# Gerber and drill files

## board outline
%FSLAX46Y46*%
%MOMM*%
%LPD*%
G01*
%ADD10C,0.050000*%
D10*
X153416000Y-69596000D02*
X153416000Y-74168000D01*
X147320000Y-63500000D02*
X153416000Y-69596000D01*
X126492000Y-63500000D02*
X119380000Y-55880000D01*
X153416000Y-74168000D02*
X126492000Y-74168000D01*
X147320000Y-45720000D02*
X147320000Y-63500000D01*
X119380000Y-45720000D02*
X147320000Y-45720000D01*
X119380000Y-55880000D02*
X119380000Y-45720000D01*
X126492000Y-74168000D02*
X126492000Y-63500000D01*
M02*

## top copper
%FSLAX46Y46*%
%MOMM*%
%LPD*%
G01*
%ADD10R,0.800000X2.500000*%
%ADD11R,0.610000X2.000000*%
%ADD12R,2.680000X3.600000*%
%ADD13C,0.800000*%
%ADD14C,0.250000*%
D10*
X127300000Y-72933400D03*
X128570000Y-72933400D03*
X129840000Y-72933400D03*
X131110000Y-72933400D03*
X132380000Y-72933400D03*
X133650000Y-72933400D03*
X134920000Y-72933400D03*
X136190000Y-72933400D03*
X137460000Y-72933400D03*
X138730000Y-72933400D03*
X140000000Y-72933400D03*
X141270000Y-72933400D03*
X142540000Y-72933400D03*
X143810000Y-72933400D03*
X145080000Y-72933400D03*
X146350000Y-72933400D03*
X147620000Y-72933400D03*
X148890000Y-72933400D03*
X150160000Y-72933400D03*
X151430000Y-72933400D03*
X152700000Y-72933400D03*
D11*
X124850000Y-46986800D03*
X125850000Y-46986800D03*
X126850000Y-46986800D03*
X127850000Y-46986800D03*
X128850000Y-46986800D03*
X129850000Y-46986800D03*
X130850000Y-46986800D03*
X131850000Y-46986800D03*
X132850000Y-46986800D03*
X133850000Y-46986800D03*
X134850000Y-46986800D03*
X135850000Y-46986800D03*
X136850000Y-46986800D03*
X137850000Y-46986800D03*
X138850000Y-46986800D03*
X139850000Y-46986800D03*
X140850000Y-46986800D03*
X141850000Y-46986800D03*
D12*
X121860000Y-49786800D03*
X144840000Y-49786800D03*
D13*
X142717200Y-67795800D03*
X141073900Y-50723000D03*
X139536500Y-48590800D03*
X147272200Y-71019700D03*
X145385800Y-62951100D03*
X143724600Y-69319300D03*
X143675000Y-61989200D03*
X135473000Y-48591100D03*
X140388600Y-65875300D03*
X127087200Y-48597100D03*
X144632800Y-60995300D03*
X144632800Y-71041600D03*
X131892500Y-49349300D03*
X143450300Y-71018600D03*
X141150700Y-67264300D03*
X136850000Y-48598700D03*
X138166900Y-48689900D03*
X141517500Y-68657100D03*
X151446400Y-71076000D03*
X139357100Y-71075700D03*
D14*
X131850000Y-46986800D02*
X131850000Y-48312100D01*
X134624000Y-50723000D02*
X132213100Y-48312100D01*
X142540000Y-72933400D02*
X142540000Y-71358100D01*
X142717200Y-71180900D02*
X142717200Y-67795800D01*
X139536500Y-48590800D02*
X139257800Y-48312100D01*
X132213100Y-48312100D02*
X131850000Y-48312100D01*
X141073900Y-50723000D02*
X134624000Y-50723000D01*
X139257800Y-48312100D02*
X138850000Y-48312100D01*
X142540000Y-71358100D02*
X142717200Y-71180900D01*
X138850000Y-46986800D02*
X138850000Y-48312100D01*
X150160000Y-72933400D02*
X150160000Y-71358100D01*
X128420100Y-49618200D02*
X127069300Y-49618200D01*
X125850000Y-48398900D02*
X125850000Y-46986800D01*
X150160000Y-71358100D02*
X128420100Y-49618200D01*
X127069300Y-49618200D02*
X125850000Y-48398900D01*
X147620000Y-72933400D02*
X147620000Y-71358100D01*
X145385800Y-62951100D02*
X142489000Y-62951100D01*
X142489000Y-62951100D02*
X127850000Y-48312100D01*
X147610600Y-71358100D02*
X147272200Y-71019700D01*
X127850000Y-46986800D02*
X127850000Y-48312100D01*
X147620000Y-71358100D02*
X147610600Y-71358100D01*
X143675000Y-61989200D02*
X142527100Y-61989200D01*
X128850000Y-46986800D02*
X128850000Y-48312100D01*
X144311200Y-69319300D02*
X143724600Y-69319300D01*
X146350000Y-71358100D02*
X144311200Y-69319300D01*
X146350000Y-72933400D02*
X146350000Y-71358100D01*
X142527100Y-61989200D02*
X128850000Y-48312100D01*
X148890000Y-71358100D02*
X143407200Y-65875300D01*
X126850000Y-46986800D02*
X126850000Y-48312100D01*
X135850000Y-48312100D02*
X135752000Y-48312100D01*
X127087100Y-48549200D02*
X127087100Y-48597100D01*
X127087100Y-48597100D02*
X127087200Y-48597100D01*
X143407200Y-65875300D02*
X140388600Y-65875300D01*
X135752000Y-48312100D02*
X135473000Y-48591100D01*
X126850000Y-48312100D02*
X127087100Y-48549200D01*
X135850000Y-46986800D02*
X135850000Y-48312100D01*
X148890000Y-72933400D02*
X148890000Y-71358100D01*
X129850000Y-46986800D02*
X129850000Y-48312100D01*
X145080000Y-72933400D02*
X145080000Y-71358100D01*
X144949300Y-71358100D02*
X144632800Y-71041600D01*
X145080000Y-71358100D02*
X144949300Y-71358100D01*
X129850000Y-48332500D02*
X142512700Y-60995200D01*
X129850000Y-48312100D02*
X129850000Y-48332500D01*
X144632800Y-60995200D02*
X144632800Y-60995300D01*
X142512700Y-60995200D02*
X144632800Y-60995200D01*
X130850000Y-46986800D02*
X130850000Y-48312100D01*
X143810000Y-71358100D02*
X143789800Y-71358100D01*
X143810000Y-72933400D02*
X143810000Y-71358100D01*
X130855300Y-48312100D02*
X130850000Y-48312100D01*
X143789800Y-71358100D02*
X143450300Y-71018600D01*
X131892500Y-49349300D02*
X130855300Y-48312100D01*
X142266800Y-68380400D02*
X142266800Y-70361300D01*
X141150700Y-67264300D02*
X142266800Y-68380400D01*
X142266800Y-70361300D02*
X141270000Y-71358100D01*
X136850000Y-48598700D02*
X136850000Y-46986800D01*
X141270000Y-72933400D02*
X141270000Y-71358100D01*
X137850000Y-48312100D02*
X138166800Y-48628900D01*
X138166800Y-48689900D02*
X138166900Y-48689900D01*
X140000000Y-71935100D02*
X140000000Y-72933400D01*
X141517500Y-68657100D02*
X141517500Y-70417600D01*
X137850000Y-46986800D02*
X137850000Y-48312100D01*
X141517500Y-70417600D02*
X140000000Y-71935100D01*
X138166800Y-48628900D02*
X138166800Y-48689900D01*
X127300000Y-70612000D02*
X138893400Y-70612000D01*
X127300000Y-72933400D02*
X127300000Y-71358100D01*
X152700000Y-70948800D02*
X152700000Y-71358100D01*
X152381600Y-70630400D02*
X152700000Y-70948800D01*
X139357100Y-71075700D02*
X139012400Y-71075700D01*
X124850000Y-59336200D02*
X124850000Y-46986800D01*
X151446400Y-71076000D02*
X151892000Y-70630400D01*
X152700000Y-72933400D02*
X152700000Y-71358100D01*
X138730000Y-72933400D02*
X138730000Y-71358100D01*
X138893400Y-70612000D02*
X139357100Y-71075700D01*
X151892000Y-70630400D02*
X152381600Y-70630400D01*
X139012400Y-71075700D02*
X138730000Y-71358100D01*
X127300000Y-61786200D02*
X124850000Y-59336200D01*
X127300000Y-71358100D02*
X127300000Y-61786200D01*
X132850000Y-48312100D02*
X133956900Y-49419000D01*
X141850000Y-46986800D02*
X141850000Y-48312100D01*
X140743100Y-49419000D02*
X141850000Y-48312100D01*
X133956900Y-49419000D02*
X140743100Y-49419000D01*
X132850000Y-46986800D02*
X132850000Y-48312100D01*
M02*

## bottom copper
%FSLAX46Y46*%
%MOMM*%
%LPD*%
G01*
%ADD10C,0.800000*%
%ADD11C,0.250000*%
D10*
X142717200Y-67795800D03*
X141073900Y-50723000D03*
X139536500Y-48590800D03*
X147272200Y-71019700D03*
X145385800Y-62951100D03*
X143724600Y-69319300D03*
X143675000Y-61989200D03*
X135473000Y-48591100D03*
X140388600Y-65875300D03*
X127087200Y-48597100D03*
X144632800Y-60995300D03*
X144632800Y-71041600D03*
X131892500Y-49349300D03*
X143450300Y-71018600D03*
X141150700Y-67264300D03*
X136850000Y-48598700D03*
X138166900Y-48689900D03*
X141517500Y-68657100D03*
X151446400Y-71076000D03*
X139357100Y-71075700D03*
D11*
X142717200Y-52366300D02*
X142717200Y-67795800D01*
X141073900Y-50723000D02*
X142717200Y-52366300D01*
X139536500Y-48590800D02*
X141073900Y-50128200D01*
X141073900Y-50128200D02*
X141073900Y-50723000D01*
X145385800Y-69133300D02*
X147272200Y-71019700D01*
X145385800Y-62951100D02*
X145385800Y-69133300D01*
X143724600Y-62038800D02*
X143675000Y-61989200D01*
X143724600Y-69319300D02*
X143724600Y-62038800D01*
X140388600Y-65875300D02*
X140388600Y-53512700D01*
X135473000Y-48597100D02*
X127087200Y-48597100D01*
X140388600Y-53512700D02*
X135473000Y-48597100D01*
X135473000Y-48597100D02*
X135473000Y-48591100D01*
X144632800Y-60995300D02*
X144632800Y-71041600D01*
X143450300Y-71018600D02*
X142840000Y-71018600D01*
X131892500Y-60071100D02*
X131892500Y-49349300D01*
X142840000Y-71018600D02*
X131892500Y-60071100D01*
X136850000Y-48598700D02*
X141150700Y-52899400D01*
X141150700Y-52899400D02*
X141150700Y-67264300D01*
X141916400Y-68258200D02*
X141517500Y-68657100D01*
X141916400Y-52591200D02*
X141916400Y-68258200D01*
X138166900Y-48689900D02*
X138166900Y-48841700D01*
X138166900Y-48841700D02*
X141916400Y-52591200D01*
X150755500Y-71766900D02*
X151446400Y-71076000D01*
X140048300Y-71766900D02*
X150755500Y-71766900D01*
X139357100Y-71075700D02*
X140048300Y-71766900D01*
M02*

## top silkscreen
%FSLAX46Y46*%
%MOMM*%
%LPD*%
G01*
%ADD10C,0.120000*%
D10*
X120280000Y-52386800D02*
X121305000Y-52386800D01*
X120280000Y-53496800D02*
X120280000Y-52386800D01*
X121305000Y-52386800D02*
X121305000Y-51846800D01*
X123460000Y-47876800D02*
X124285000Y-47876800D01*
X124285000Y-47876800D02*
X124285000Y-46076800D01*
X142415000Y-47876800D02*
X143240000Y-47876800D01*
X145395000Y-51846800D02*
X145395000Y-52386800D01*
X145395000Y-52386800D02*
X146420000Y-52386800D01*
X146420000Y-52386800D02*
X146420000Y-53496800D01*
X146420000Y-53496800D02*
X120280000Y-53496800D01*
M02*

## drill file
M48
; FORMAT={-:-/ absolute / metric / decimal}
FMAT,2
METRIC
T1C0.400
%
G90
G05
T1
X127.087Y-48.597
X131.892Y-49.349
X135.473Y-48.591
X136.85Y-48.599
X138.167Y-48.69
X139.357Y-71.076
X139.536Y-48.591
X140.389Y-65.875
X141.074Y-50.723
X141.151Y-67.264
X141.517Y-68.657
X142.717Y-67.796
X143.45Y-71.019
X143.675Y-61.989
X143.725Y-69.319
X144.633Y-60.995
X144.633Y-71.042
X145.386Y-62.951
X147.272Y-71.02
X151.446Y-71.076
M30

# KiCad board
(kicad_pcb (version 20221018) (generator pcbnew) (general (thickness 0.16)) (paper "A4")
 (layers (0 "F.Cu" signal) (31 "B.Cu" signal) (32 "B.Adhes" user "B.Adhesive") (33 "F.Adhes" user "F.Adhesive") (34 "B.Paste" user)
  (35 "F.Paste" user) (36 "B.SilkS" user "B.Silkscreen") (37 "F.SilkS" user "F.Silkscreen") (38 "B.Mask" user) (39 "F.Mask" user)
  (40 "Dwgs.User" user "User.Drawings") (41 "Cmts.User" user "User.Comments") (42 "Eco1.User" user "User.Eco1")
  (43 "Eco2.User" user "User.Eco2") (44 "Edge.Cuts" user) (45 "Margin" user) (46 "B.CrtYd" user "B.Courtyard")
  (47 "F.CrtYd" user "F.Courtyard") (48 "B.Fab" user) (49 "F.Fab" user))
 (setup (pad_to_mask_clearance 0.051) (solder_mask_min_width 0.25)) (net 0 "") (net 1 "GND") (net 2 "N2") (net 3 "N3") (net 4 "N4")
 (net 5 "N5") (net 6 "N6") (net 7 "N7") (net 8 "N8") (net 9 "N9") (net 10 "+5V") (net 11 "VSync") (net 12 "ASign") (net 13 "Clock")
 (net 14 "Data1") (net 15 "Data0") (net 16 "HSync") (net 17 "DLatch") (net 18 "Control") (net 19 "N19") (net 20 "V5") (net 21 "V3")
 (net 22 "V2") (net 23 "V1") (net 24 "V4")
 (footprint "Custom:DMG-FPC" (layer "F.Cu") (at 140 72.9334)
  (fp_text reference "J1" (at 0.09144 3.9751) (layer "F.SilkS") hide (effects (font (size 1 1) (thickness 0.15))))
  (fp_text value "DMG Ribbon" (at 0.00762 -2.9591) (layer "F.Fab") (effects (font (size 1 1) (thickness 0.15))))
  (pad "1" smd rect (at -12.7 0) (size 0.8 2.5) (layers "F.Cu" "F.Paste" "F.Mask") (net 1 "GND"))
  (pad "2" smd rect (at -11.43 0) (size 0.8 2.5) (layers "F.Cu" "F.Paste" "F.Mask") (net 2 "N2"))
  (pad "3" smd rect (at -10.16 0) (size 0.8 2.5) (layers "F.Cu" "F.Paste" "F.Mask") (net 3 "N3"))
  (pad "4" smd rect (at -8.89 0) (size 0.8 2.5) (layers "F.Cu" "F.Paste" "F.Mask") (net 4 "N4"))
  (pad "5" smd rect (at -7.62 0) (size 0.8 2.5) (layers "F.Cu" "F.Paste" "F.Mask") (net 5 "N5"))
  (pad "6" smd rect (at -6.35 0) (size 0.8 2.5) (layers "F.Cu" "F.Paste" "F.Mask") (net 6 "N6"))
  (pad "7" smd rect (at -5.08 0) (size 0.8 2.5) (layers "F.Cu" "F.Paste" "F.Mask") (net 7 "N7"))
  (pad "8" smd rect (at -3.81 0) (size 0.8 2.5) (layers "F.Cu" "F.Paste" "F.Mask") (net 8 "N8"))
  (pad "9" smd rect (at -2.54 0) (size 0.8 2.5) (layers "F.Cu" "F.Paste" "F.Mask") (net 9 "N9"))
  (pad "10" smd rect (at -1.27 0) (size 0.8 2.5) (layers "F.Cu" "F.Paste" "F.Mask") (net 1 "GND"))
  (pad "11" smd rect (at 0 0) (size 0.8 2.5) (layers "F.Cu" "F.Paste" "F.Mask") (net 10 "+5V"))
  (pad "12" smd rect (at 1.27 0) (size 0.8 2.5) (layers "F.Cu" "F.Paste" "F.Mask") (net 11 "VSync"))
  (pad "13" smd rect (at 2.54 0) (size 0.8 2.5) (layers "F.Cu" "F.Paste" "F.Mask") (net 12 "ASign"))
  (pad "14" smd rect (at 3.81 0) (size 0.8 2.5) (layers "F.Cu" "F.Paste" "F.Mask") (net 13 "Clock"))
  (pad "15" smd rect (at 5.08 0) (size 0.8 2.5) (layers "F.Cu" "F.Paste" "F.Mask") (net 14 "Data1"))
  (pad "16" smd rect (at 6.35 0) (size 0.8 2.5) (layers "F.Cu" "F.Paste" "F.Mask") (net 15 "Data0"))
  (pad "17" smd rect (at 7.62 0) (size 0.8 2.5) (layers "F.Cu" "F.Paste" "F.Mask") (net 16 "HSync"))
  (pad "18" smd rect (at 8.89 0) (size 0.8 2.5) (layers "F.Cu" "F.Paste" "F.Mask") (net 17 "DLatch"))
  (pad "19" smd rect (at 10.16 0) (size 0.8 2.5) (layers "F.Cu" "F.Paste" "F.Mask") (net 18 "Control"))
  (pad "20" smd rect (at 11.43 0) (size 0.8 2.5) (layers "F.Cu" "F.Paste" "F.Mask") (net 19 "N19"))
  (pad "21" smd rect (at 12.7 0) (size 0.8 2.5) (layers "F.Cu" "F.Paste" "F.Mask") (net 1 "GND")))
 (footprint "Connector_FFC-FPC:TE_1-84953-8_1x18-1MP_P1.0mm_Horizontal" (layer "F.Cu") (at 133.35 48.7868)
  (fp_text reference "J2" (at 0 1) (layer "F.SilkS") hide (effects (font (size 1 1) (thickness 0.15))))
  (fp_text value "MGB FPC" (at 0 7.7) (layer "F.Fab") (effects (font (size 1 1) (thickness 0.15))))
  (fp_line (start -13.07 3.6) (end -12.045 3.6) (stroke (width 0.12) (type solid)) (layer "F.SilkS"))
  (fp_line (start -13.07 4.71) (end -13.07 3.6) (stroke (width 0.12) (type solid)) (layer "F.SilkS"))
  (fp_line (start -12.045 3.6) (end -12.045 3.06) (stroke (width 0.12) (type solid)) (layer "F.SilkS"))
  (fp_line (start -9.89 -0.91) (end -9.065 -0.91) (stroke (width 0.12) (type solid)) (layer "F.SilkS"))
  (fp_line (start -9.065 -0.91) (end -9.065 -2.71) (stroke (width 0.12) (type solid)) (layer "F.SilkS"))
  (fp_line (start 9.065 -0.91) (end 9.89 -0.91) (stroke (width 0.12) (type solid)) (layer "F.SilkS"))
  (fp_line (start 12.045 3.06) (end 12.045 3.6) (stroke (width 0.12) (type solid)) (layer "F.SilkS"))
  (fp_line (start 12.045 3.6) (end 13.07 3.6) (stroke (width 0.12) (type solid)) (layer "F.SilkS"))
  (fp_line (start 13.07 3.6) (end 13.07 4.71) (stroke (width 0.12) (type solid)) (layer "F.SilkS"))
  (fp_line (start 13.07 4.71) (end -13.07 4.71) (stroke (width 0.12) (type solid)) (layer "F.SilkS"))
  (pad "1" smd rect (at -8.5 -1.8) (size 0.61 2) (layers "F.Cu" "F.Paste" "F.Mask") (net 1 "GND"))
  (pad "2" smd rect (at -7.5 -1.8) (size 0.61 2) (layers "F.Cu" "F.Paste" "F.Mask") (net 18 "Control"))
  (pad "3" smd rect (at -6.5 -1.8) (size 0.61 2) (layers "F.Cu" "F.Paste" "F.Mask") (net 17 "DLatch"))
  (pad "4" smd rect (at -5.5 -1.8) (size 0.61 2) (layers "F.Cu" "F.Paste" "F.Mask") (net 16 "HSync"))
  (pad "5" smd rect (at -4.5 -1.8) (size 0.61 2) (layers "F.Cu" "F.Paste" "F.Mask") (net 15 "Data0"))
  (pad "6" smd rect (at -3.5 -1.8) (size 0.61 2) (layers "F.Cu" "F.Paste" "F.Mask") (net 14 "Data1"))
  (pad "7" smd rect (at -2.5 -1.8) (size 0.61 2) (layers "F.Cu" "F.Paste" "F.Mask") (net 13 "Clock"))
  (pad "8" smd rect (at -1.5 -1.8) (size 0.61 2) (layers "F.Cu" "F.Paste" "F.Mask") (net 12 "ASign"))
  (pad "9" smd rect (at -0.5 -1.8) (size 0.61 2) (layers "F.Cu" "F.Paste" "F.Mask") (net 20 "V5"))
  (pad "10" smd rect (at 0.5 -1.8) (size 0.61 2) (layers "F.Cu" "F.Paste" "F.Mask") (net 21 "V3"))
  (pad "11" smd rect (at 1.5 -1.8) (size 0.61 2) (layers "F.Cu" "F.Paste" "F.Mask") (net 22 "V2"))
  (pad "12" smd rect (at 2.5 -1.8) (size 0.61 2) (layers "F.Cu" "F.Paste" "F.Mask") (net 17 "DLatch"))
  (pad "13" smd rect (at 3.5 -1.8) (size 0.61 2) (layers "F.Cu" "F.Paste" "F.Mask") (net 11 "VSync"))
  (pad "14" smd rect (at 4.5 -1.8) (size 0.61 2) (layers "F.Cu" "F.Paste" "F.Mask") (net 10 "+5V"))
  (pad "15" smd rect (at 5.5 -1.8) (size 0.61 2) (layers "F.Cu" "F.Paste" "F.Mask") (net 12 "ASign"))
  (pad "16" smd rect (at 6.5 -1.8) (size 0.61 2) (layers "F.Cu" "F.Paste" "F.Mask") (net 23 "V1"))
  (pad "17" smd rect (at 7.5 -1.8) (size 0.61 2) (layers "F.Cu" "F.Paste" "F.Mask") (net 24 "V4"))
  (pad "18" smd rect (at 8.5 -1.8) (size 0.61 2) (layers "F.Cu" "F.Paste" "F.Mask") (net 20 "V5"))
  (pad "MP" smd rect (at -11.49 1) (size 2.68 3.6) (layers "F.Cu" "F.Paste" "F.Mask"))
  (pad "MP" smd rect (at 11.49 1) (size 2.68 3.6) (layers "F.Cu" "F.Paste" "F.Mask")))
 (gr_line (start 153.416 69.596) (end 153.416 74.168) (stroke (width 0.05) (type solid)) (layer "Edge.Cuts"))
 (gr_line (start 147.32 63.5) (end 153.416 69.596) (stroke (width 0.05) (type solid)) (layer "Edge.Cuts"))
 (gr_line (start 126.492 63.5) (end 119.38 55.88) (stroke (width 0.05) (type solid)) (layer "Edge.Cuts"))
 (gr_line (start 153.416 74.168) (end 126.492 74.168) (stroke (width 0.05) (type solid)) (layer "Edge.Cuts"))
 (gr_line (start 147.32 45.72) (end 147.32 63.5) (stroke (width 0.05) (type solid)) (layer "Edge.Cuts"))
 (gr_line (start 119.38 45.72) (end 147.32 45.72) (stroke (width 0.05) (type solid)) (layer "Edge.Cuts"))
 (gr_line (start 119.38 55.88) (end 119.38 45.72) (stroke (width 0.05) (type solid)) (layer "Edge.Cuts"))
 (gr_line (start 126.492 74.168) (end 126.492 63.5) (stroke (width 0.05) (type solid)) (layer "Edge.Cuts"))
 (segment (start 131.85 46.9868) (end 131.85 48.3121) (width 0.25) (layer "F.Cu") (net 12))
 (segment (start 134.624 50.723) (end 132.2131 48.3121) (width 0.25) (layer "F.Cu") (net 12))
 (segment (start 142.54 72.9334) (end 142.54 71.3581) (width 0.25) (layer "F.Cu") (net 12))
 (segment (start 142.7172 71.1809) (end 142.7172 67.7958) (width 0.25) (layer "F.Cu") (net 12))
 (segment (start 139.5365 48.5908) (end 139.2578 48.3121) (width 0.25) (layer "F.Cu") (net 12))
 (segment (start 132.2131 48.3121) (end 131.85 48.3121) (width 0.25) (layer "F.Cu") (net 12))
 (segment (start 141.0739 50.723) (end 134.624 50.723) (width 0.25) (layer "F.Cu") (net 12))
 (segment (start 139.2578 48.3121) (end 138.85 48.3121) (width 0.25) (layer "F.Cu") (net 12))
 (segment (start 142.54 71.3581) (end 142.7172 71.1809) (width 0.25) (layer "F.Cu") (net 12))
 (segment (start 138.85 46.9868) (end 138.85 48.3121) (width 0.25) (layer "F.Cu") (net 12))
 (via (at 142.7172 67.7958) (size 0.8) (drill 0.4) (layers "F.Cu" "B.Cu") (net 12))
 (via (at 141.0739 50.723) (size 0.8) (drill 0.4) (layers "F.Cu" "B.Cu") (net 12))
 (via (at 139.5365 48.5908) (size 0.8) (drill 0.4) (layers "F.Cu" "B.Cu") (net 12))
 (segment (start 142.7172 52.3663) (end 142.7172 67.7958) (width 0.25) (layer "B.Cu") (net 12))
 (segment (start 141.0739 50.723) (end 142.7172 52.3663) (width 0.25) (layer "B.Cu") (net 12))
 (segment (start 139.5365 48.5908) (end 141.0739 50.1282) (width 0.25) (layer "B.Cu") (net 12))
 (segment (start 141.0739 50.1282) (end 141.0739 50.723) (width 0.25) (layer "B.Cu") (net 12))
 (segment (start 150.16 72.9334) (end 150.16 71.3581) (width 0.25) (layer "F.Cu") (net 18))
 (segment (start 128.4201 49.6182) (end 127.0693 49.6182) (width 0.25) (layer "F.Cu") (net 18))
 (segment (start 125.85 48.3989) (end 125.85 46.9868) (width 0.25) (layer "F.Cu") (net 18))
 (segment (start 150.16 71.3581) (end 128.4201 49.6182) (width 0.25) (layer "F.Cu") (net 18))
 (segment (start 127.0693 49.6182) (end 125.85 48.3989) (width 0.25) (layer "F.Cu") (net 18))
 (segment (start 147.62 72.9334) (end 147.62 71.3581) (width 0.25) (layer "F.Cu") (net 16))
 (segment (start 145.3858 62.9511) (end 142.489 62.9511) (width 0.25) (layer "F.Cu") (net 16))
 (segment (start 142.489 62.9511) (end 127.85 48.3121) (width 0.25) (layer "F.Cu") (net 16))
 (segment (start 147.6106 71.3581) (end 147.2722 71.0197) (width 0.25) (layer "F.Cu") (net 16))
 (segment (start 127.85 46.9868) (end 127.85 48.3121) (width 0.25) (layer "F.Cu") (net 16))
 (segment (start 147.62 71.3581) (end 147.6106 71.3581) (width 0.25) (layer "F.Cu") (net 16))
 (via (at 147.2722 71.0197) (size 0.8) (drill 0.4) (layers "F.Cu" "B.Cu") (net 16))
 (via (at 145.3858 62.9511) (size 0.8) (drill 0.4) (layers "F.Cu" "B.Cu") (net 16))
 (segment (start 145.3858 69.1333) (end 147.2722 71.0197) (width 0.25) (layer "B.Cu") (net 16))
 (segment (start 145.3858 62.9511) (end 145.3858 69.1333) (width 0.25) (layer "B.Cu") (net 16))
 (segment (start 143.675 61.9892) (end 142.5271 61.9892) (width 0.25) (layer "F.Cu") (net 15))
 (segment (start 128.85 46.9868) (end 128.85 48.3121) (width 0.25) (layer "F.Cu") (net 15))
 (segment (start 144.3112 69.3193) (end 143.7246 69.3193) (width 0.25) (layer "F.Cu") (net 15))
 (segment (start 146.35 71.3581) (end 144.3112 69.3193) (width 0.25) (layer "F.Cu") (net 15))
 (segment (start 146.35 72.9334) (end 146.35 71.3581) (width 0.25) (layer "F.Cu") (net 15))
 (segment (start 142.5271 61.9892) (end 128.85 48.3121) (width 0.25) (layer "F.Cu") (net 15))
 (via (at 143.7246 69.3193) (size 0.8) (drill 0.4) (layers "F.Cu" "B.Cu") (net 15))
 (via (at 143.675 61.9892) (size 0.8) (drill 0.4) (layers "F.Cu" "B.Cu") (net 15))
 (segment (start 143.7246 62.0388) (end 143.675 61.9892) (width 0.25) (layer "B.Cu") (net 15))
 (segment (start 143.7246 69.3193) (end 143.7246 62.0388) (width 0.25) (layer "B.Cu") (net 15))
 (segment (start 148.89 71.3581) (end 143.4072 65.8753) (width 0.25) (layer "F.Cu") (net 17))
 (segment (start 126.85 46.9868) (end 126.85 48.3121) (width 0.25) (layer "F.Cu") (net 17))
 (segment (start 135.85 48.3121) (end 135.752 48.3121) (width 0.25) (layer "F.Cu") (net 17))
 (segment (start 127.0871 48.5492) (end 127.0871 48.5971) (width 0.25) (layer "F.Cu") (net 17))
 (segment (start 127.0871 48.5971) (end 127.0872 48.5971) (width 0.25) (layer "F.Cu") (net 17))
 (segment (start 143.4072 65.8753) (end 140.3886 65.8753) (width 0.25) (layer "F.Cu") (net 17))
 (segment (start 135.752 48.3121) (end 135.473 48.5911) (width 0.25) (layer "F.Cu") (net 17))
 (segment (start 126.85 48.3121) (end 127.0871 48.5492) (width 0.25) (layer "F.Cu") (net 17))
 (segment (start 135.85 46.9868) (end 135.85 48.3121) (width 0.25) (layer "F.Cu") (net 17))
 (segment (start 148.89 72.9334) (end 148.89 71.3581) (width 0.25) (layer "F.Cu") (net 17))
 (via (at 135.473 48.5911) (size 0.8) (drill 0.4) (layers "F.Cu" "B.Cu") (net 17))
 (via (at 140.3886 65.8753) (size 0.8) (drill 0.4) (layers "F.Cu" "B.Cu") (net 17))
 (via (at 127.0872 48.5971) (size 0.8) (drill 0.4) (layers "F.Cu" "B.Cu") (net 17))
 (segment (start 140.3886 65.8753) (end 140.3886 53.5127) (width 0.25) (layer "B.Cu") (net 17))
 (segment (start 135.473 48.5971) (end 127.0872 48.5971) (width 0.25) (layer "B.Cu") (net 17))
 (segment (start 140.3886 53.5127) (end 135.473 48.5971) (width 0.25) (layer "B.Cu") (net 17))
 (segment (start 135.473 48.5971) (end 135.473 48.5911) (width 0.25) (layer "B.Cu") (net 17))
 (segment (start 129.85 46.9868) (end 129.85 48.3121) (width 0.25) (layer "F.Cu") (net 14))
 (segment (start 145.08 72.9334) (end 145.08 71.3581) (width 0.25) (layer "F.Cu") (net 14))
 (segment (start 144.9493 71.3581) (end 144.6328 71.0416) (width 0.25) (layer "F.Cu") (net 14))
 (segment (start 145.08 71.3581) (end 144.9493 71.3581) (width 0.25) (layer "F.Cu") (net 14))
 (segment (start 129.85 48.3325) (end 142.5127 60.9952) (width 0.25) (layer "F.Cu") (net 14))
 (segment (start 129.85 48.3121) (end 129.85 48.3325) (width 0.25) (layer "F.Cu") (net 14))
 (segment (start 144.6328 60.9952) (end 144.6328 60.9953) (width 0.25) (layer "F.Cu") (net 14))
 (segment (start 142.5127 60.9952) (end 144.6328 60.9952) (width 0.25) (layer "F.Cu") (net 14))
 (via (at 144.6328 60.9953) (size 0.8) (drill 0.4) (layers "F.Cu" "B.Cu") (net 14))
 (via (at 144.6328 71.0416) (size 0.8) (drill 0.4) (layers "F.Cu" "B.Cu") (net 14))
 (segment (start 144.6328 60.9953) (end 144.6328 71.0416) (width 0.25) (layer "B.Cu") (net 14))
 (segment (start 130.85 46.9868) (end 130.85 48.3121) (width 0.25) (layer "F.Cu") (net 13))
 (segment (start 143.81 71.3581) (end 143.7898 71.3581) (width 0.25) (layer "F.Cu") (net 13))
 (segment (start 143.81 72.9334) (end 143.81 71.3581) (width 0.25) (layer "F.Cu") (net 13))
 (segment (start 130.8553 48.3121) (end 130.85 48.3121) (width 0.25) (layer "F.Cu") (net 13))
 (segment (start 143.7898 71.3581) (end 143.4503 71.0186) (width 0.25) (layer "F.Cu") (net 13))
 (segment (start 131.8925 49.3493) (end 130.8553 48.3121) (width 0.25) (layer "F.Cu") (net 13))
 (via (at 131.8925 49.3493) (size 0.8) (drill 0.4) (layers "F.Cu" "B.Cu") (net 13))
 (via (at 143.4503 71.0186) (size 0.8) (drill 0.4) (layers "F.Cu" "B.Cu") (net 13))
 (segment (start 143.4503 71.0186) (end 142.84 71.0186) (width 0.25) (layer "B.Cu") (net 13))
 (segment (start 131.8925 60.0711) (end 131.8925 49.3493) (width 0.25) (layer "B.Cu") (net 13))
 (segment (start 142.84 71.0186) (end 131.8925 60.0711) (width 0.25) (layer "B.Cu") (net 13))
 (segment (start 142.2668 68.3804) (end 142.2668 70.3613) (width 0.25) (layer "F.Cu") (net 11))
 (segment (start 141.1507 67.2643) (end 142.2668 68.3804) (width 0.25) (layer "F.Cu") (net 11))
 (segment (start 142.2668 70.3613) (end 141.27 71.3581) (width 0.25) (layer "F.Cu") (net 11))
 (segment (start 136.85 48.5987) (end 136.85 46.9868) (width 0.25) (layer "F.Cu") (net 11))
 (segment (start 141.27 72.9334) (end 141.27 71.3581) (width 0.25) (layer "F.Cu") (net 11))
 (via (at 141.1507 67.2643) (size 0.8) (drill 0.4) (layers "F.Cu" "B.Cu") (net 11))
 (via (at 136.85 48.5987) (size 0.8) (drill 0.4) (layers "F.Cu" "B.Cu") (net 11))
 (segment (start 136.85 48.5987) (end 141.1507 52.8994) (width 0.25) (layer "B.Cu") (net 11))
 (segment (start 141.1507 52.8994) (end 141.1507 67.2643) (width 0.25) (layer "B.Cu") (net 11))
 (segment (start 137.85 48.3121) (end 138.1668 48.6289) (width 0.25) (layer "F.Cu") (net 10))
 (segment (start 138.1668 48.6899) (end 138.1669 48.6899) (width 0.25) (layer "F.Cu") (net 10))
 (segment (start 140 71.9351) (end 140 72.9334) (width 0.25) (layer "F.Cu") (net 10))
 (segment (start 141.5175 68.6571) (end 141.5175 70.4176) (width 0.25) (layer "F.Cu") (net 10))
 (segment (start 137.85 46.9868) (end 137.85 48.3121) (width 0.25) (layer "F.Cu") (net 10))
 (segment (start 141.5175 70.4176) (end 140 71.9351) (width 0.25) (layer "F.Cu") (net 10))
 (segment (start 138.1668 48.6289) (end 138.1668 48.6899) (width 0.25) (layer "F.Cu") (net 10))
 (via (at 138.1669 48.6899) (size 0.8) (drill 0.4) (layers "F.Cu" "B.Cu") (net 10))
 (via (at 141.5175 68.6571) (size 0.8) (drill 0.4) (layers "F.Cu" "B.Cu") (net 10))
 (segment (start 141.9164 68.2582) (end 141.5175 68.6571) (width 0.25) (layer "B.Cu") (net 10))
 (segment (start 141.9164 52.5912) (end 141.9164 68.2582) (width 0.25) (layer "B.Cu") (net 10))
 (segment (start 138.1669 48.6899) (end 138.1669 48.8417) (width 0.25) (layer "B.Cu") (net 10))
 (segment (start 138.1669 48.8417) (end 141.9164 52.5912) (width 0.25) (layer "B.Cu") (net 10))
 (segment (start 127.3 70.612) (end 138.8934 70.612) (width 0.25) (layer "F.Cu") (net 1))
 (segment (start 127.3 72.9334) (end 127.3 71.3581) (width 0.25) (layer "F.Cu") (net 1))
 (segment (start 152.7 70.9488) (end 152.7 71.3581) (width 0.25) (layer "F.Cu") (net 1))
 (segment (start 152.3816 70.6304) (end 152.7 70.9488) (width 0.25) (layer "F.Cu") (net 1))
 (segment (start 139.3571 71.0757) (end 139.0124 71.0757) (width 0.25) (layer "F.Cu") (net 1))
 (segment (start 124.85 59.3362) (end 124.85 46.9868) (width 0.25) (layer "F.Cu") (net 1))
 (segment (start 151.4464 71.076) (end 151.892 70.6304) (width 0.25) (layer "F.Cu") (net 1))
 (segment (start 152.7 72.9334) (end 152.7 71.3581) (width 0.25) (layer "F.Cu") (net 1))
 (segment (start 138.73 72.9334) (end 138.73 71.3581) (width 0.25) (layer "F.Cu") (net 1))
 (segment (start 138.8934 70.612) (end 139.3571 71.0757) (width 0.25) (layer "F.Cu") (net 1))
 (segment (start 151.892 70.6304) (end 152.3816 70.6304) (width 0.25) (layer "F.Cu") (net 1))
 (segment (start 139.0124 71.0757) (end 138.73 71.3581) (width 0.25) (layer "F.Cu") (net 1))
 (segment (start 127.3 61.7862) (end 124.85 59.3362) (width 0.25) (layer "F.Cu") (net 1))
 (segment (start 127.3 71.3581) (end 127.3 61.7862) (width 0.25) (layer "F.Cu") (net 1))
 (via (at 151.4464 71.076) (size 0.8) (drill 0.4) (layers "F.Cu" "B.Cu") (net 1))
 (via (at 139.3571 71.0757) (size 0.8) (drill 0.4) (layers "F.Cu" "B.Cu") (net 1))
 (segment (start 150.7555 71.7669) (end 151.4464 71.076) (width 0.25) (layer "B.Cu") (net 1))
 (segment (start 140.0483 71.7669) (end 150.7555 71.7669) (width 0.25) (layer "B.Cu") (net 1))
 (segment (start 139.3571 71.0757) (end 140.0483 71.7669) (width 0.25) (layer "B.Cu") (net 1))
 (segment (start 132.85 48.3121) (end 133.9569 49.419) (width 0.25) (layer "F.Cu") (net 20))
 (segment (start 141.85 46.9868) (end 141.85 48.3121) (width 0.25) (layer "F.Cu") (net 20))
 (segment (start 140.7431 49.419) (end 141.85 48.3121) (width 0.25) (layer "F.Cu") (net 20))
 (segment (start 133.9569 49.419) (end 140.7431 49.419) (width 0.25) (layer "F.Cu") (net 20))
 (segment (start 132.85 46.9868) (end 132.85 48.3121) (width 0.25) (layer "F.Cu") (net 20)))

